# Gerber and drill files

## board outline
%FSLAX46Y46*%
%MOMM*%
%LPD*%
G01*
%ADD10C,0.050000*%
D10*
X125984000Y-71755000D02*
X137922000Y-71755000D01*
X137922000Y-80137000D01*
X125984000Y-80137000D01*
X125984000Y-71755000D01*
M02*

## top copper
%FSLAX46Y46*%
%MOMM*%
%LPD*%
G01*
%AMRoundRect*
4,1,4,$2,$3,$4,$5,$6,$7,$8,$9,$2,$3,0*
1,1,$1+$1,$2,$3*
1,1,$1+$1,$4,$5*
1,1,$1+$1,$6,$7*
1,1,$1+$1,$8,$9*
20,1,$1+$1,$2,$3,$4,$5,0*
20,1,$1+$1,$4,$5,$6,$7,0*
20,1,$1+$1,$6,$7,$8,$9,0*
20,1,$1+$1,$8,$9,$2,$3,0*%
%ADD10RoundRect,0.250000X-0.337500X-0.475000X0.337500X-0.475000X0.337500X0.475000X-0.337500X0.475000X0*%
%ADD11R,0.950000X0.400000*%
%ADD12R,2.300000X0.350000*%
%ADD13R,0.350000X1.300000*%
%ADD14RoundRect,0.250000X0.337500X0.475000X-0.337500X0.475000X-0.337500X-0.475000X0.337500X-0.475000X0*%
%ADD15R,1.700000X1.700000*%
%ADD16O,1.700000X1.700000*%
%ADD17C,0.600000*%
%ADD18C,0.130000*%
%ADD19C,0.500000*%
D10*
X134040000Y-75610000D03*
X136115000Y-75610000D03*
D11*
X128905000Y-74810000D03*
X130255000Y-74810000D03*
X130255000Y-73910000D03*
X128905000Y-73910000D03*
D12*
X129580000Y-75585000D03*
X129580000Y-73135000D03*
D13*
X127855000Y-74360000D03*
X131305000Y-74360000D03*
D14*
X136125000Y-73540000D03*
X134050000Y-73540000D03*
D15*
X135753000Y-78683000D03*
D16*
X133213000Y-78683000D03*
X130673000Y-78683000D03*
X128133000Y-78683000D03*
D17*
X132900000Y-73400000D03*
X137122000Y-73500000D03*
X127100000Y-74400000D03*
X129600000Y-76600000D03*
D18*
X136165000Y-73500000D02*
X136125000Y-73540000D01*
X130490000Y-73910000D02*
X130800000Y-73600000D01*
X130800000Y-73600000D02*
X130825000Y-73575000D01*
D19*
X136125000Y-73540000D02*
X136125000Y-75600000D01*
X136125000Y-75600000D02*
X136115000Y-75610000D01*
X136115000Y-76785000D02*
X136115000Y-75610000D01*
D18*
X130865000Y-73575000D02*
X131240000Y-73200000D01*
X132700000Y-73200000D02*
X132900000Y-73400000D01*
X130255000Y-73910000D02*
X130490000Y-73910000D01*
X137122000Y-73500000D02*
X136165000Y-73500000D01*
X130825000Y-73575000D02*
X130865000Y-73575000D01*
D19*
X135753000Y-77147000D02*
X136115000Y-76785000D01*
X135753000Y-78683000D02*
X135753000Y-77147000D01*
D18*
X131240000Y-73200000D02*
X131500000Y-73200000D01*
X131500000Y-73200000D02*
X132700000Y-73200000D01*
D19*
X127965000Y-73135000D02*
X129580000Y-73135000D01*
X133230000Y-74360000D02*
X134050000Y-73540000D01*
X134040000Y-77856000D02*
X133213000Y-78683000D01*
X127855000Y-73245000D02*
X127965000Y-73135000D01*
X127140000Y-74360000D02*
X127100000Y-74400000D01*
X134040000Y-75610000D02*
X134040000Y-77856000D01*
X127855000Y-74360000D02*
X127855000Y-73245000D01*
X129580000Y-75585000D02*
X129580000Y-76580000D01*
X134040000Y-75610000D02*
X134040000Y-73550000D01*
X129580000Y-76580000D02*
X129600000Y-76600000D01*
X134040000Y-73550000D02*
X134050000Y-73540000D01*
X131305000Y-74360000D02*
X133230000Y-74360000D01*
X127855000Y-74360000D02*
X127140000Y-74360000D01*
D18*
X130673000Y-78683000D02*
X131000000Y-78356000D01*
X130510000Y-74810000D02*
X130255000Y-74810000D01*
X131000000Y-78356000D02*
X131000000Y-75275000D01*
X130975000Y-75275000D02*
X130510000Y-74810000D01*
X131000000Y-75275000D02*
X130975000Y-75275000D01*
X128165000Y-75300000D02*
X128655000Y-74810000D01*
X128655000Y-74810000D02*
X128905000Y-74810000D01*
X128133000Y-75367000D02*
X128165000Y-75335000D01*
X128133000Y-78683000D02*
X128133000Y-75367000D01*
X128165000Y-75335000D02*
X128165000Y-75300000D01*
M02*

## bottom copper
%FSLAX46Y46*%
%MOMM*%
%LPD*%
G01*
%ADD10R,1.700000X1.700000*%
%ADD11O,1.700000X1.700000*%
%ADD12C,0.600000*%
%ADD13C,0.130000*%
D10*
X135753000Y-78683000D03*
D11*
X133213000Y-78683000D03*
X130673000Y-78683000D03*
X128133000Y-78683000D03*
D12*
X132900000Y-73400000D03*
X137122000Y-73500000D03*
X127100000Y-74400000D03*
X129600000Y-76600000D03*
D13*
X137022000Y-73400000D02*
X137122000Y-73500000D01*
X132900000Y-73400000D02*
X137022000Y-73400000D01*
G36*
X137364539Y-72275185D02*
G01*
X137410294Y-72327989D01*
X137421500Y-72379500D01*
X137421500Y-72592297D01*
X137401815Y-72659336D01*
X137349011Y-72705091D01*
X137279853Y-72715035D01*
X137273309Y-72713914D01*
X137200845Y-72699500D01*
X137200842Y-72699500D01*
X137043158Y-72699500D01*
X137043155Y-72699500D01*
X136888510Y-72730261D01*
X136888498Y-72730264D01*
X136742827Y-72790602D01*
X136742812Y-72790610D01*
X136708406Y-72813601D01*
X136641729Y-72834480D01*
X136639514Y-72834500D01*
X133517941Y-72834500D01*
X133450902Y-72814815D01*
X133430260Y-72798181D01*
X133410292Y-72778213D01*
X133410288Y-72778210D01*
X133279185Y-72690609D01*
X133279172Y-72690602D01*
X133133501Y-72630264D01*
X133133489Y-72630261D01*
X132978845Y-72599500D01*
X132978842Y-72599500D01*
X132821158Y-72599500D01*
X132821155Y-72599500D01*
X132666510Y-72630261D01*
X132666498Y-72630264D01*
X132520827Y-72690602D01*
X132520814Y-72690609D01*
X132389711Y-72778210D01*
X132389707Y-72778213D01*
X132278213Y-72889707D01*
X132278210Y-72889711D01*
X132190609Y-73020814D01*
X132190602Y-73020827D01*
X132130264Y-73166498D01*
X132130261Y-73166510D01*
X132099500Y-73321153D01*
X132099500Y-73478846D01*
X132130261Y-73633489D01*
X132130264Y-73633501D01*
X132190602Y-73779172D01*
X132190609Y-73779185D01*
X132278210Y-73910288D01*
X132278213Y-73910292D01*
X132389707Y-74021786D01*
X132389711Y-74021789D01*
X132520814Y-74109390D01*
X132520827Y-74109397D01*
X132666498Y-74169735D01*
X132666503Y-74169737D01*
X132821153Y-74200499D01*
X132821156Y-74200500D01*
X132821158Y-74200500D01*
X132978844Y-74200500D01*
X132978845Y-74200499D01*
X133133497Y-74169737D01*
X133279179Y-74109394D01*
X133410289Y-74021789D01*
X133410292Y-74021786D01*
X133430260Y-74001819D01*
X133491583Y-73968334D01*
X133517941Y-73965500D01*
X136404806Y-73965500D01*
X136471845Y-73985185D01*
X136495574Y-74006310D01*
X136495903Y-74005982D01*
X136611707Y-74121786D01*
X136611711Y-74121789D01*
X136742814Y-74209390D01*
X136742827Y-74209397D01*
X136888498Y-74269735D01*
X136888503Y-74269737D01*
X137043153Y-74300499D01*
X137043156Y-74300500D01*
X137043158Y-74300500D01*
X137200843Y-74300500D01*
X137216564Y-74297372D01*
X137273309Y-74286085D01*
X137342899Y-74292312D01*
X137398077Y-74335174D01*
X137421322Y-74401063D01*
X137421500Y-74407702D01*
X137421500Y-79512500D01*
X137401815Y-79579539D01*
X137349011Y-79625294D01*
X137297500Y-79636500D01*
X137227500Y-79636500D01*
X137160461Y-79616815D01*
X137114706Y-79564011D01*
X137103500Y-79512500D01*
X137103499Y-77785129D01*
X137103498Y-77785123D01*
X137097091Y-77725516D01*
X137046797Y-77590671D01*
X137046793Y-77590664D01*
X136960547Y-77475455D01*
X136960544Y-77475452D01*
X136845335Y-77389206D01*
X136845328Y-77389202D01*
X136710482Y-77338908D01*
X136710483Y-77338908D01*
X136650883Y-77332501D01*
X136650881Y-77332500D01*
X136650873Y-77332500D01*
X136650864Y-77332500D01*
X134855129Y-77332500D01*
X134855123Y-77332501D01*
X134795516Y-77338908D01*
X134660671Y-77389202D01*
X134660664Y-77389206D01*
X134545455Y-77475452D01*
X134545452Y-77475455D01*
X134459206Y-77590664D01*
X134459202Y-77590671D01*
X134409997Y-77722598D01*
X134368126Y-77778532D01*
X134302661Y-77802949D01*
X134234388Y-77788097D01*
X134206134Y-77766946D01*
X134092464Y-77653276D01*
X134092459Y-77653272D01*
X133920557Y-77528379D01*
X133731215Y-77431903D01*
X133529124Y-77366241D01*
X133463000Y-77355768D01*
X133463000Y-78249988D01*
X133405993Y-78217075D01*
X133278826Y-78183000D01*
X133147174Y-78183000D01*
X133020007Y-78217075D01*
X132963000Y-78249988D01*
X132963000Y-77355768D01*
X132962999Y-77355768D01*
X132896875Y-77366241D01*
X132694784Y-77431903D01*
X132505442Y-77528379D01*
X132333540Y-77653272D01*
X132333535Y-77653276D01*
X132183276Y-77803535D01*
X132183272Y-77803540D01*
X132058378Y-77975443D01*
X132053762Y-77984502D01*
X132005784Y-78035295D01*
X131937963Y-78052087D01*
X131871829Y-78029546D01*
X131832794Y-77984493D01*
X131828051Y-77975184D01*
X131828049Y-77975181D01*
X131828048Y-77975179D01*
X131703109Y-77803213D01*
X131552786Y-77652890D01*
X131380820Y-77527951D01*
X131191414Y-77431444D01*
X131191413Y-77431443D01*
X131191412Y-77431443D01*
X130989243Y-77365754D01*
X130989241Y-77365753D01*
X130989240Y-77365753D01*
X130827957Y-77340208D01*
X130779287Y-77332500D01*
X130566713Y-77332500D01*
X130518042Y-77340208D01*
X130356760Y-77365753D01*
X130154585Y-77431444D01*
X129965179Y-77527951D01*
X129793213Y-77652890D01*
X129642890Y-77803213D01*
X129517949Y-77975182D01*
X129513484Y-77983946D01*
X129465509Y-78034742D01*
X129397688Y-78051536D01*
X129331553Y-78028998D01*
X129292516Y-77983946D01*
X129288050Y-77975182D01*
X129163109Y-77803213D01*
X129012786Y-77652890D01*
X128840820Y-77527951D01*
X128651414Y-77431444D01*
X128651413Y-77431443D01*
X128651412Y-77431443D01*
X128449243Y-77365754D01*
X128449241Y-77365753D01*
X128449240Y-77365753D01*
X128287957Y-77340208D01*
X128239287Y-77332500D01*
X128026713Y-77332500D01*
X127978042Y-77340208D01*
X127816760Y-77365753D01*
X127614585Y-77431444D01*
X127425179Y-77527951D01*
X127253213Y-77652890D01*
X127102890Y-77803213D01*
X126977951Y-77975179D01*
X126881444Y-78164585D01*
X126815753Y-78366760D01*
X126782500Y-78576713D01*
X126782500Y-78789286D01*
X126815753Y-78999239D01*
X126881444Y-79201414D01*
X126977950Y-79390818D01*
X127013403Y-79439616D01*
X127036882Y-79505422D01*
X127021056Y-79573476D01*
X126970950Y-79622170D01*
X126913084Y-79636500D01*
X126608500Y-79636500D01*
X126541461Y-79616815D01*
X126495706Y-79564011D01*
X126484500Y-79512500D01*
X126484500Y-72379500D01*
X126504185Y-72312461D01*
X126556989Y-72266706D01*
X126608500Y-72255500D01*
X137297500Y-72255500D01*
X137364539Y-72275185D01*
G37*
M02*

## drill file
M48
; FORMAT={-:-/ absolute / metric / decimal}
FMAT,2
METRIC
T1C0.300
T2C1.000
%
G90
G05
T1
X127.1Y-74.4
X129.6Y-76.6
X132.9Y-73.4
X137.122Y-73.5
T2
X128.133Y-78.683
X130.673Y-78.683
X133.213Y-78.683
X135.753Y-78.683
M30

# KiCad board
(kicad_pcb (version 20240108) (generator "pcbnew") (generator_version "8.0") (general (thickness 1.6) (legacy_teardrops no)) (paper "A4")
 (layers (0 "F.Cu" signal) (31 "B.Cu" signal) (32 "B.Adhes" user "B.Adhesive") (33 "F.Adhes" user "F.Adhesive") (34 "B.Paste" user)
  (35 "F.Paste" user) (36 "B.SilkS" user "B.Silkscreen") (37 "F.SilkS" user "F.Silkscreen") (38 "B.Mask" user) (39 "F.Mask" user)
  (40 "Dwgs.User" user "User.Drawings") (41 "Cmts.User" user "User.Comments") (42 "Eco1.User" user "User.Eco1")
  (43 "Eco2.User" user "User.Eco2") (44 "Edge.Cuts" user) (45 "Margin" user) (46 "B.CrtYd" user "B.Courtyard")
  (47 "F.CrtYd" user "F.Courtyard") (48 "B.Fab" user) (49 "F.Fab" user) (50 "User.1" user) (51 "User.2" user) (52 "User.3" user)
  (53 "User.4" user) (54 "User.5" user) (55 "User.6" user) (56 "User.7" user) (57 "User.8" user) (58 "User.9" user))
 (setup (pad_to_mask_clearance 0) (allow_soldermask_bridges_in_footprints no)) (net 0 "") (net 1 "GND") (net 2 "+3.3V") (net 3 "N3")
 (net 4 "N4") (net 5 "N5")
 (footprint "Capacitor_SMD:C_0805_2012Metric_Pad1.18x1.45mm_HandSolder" (layer "F.Cu") (at 135.0775 75.61)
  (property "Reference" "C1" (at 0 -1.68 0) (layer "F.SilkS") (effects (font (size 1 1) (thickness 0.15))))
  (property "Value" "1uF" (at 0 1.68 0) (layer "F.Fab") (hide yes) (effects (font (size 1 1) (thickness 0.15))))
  (pad "1" smd roundrect (at -1.0375 0) (size 1.175 1.45) (layers "F.Cu" "F.Paste" "F.Mask") (roundrect_rratio 0.212766) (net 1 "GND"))
  (pad "2" smd roundrect (at 1.0375 0) (size 1.175 1.45) (layers "F.Cu" "F.Paste" "F.Mask") (roundrect_rratio 0.212766) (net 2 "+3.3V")))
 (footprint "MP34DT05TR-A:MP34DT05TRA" (layer "F.Cu") (at 129.58 74.36 90)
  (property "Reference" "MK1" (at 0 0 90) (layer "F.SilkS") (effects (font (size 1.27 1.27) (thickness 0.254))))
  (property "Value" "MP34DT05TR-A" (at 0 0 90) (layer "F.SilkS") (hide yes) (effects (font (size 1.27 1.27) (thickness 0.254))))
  (pad "1" smd rect (at -0.45 -0.675 90) (size 0.4 0.95) (layers "F.Cu" "F.Paste" "F.Mask") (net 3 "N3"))
  (pad "2" smd rect (at -0.45 0.675 90) (size 0.4 0.95) (layers "F.Cu" "F.Paste" "F.Mask") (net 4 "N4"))
  (pad "3" smd rect (at 0.45 0.675 90) (size 0.4 0.95) (layers "F.Cu" "F.Paste" "F.Mask") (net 2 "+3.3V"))
  (pad "4" smd rect (at 0.45 -0.675 90) (size 0.4 0.95) (layers "F.Cu" "F.Paste" "F.Mask") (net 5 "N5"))
  (pad "5" smd rect (at -1.225 0 90) (size 0.35 2.3) (layers "F.Cu" "F.Paste" "F.Mask") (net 1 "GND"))
  (pad "6" smd rect (at 1.225 0 90) (size 0.35 2.3) (layers "F.Cu" "F.Paste" "F.Mask") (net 1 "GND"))
  (pad "7" smd rect (at 0 -1.725 180) (size 0.35 1.3) (layers "F.Cu" "F.Paste" "F.Mask") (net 1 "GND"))
  (pad "8" smd rect (at 0 1.725 180) (size 0.35 1.3) (layers "F.Cu" "F.Paste" "F.Mask") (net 1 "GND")))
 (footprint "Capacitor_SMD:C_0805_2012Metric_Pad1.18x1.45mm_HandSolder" (layer "F.Cu") (at 135.0875 73.54 180)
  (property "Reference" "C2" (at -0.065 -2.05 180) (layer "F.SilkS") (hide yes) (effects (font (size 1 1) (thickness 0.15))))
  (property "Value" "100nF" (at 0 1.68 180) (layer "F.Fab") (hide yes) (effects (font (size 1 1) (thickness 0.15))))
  (pad "1" smd roundrect (at -1.0375 0 180) (size 1.175 1.45) (layers "F.Cu" "F.Paste" "F.Mask") (roundrect_rratio 0.212766) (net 2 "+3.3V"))
  (pad "2" smd roundrect (at 1.0375 0 180) (size 1.175 1.45) (layers "F.Cu" "F.Paste" "F.Mask") (roundrect_rratio 0.212766) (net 1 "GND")))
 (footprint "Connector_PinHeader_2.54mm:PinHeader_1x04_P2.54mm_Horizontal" (layer "F.Cu") (at 135.753 78.683 -90)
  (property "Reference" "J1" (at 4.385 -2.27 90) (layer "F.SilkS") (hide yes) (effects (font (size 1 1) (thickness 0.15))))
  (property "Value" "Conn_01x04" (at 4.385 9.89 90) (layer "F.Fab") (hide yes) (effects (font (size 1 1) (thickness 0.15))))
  (pad "1" thru_hole rect (at 0 0 270) (size 1.7 1.7) (drill 1) (layers "*.Cu" "*.Mask") (remove_unused_layers no) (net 2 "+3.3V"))
  (pad "2" thru_hole oval (at 0 2.54 270) (size 1.7 1.7) (drill 1) (layers "*.Cu" "*.Mask") (remove_unused_layers no) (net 1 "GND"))
  (pad "3" thru_hole oval (at 0 5.08 270) (size 1.7 1.7) (drill 1) (layers "*.Cu" "*.Mask") (remove_unused_layers no) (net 4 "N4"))
  (pad "4" thru_hole oval (at 0 7.62 270) (size 1.7 1.7) (drill 1) (layers "*.Cu" "*.Mask") (remove_unused_layers no) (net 3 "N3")))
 (gr_rect (start 125.984 71.755) (end 137.922 80.137) (stroke (width 0.05) (type default)) (fill none) (layer "Edge.Cuts"))
 (segment (start 136.165 73.5) (end 136.125 73.54) (width 0.13) (layer "F.Cu") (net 2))
 (segment (start 130.49 73.91) (end 130.8 73.6) (width 0.13) (layer "F.Cu") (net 2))
 (segment (start 130.8 73.6) (end 130.825 73.575) (width 0.13) (layer "F.Cu") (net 2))
 (segment (start 136.125 73.54) (end 136.125 75.6) (width 0.5) (layer "F.Cu") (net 2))
 (segment (start 136.125 75.6) (end 136.115 75.61) (width 0.5) (layer "F.Cu") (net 2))
 (segment (start 136.115 76.785) (end 136.115 75.61) (width 0.5) (layer "F.Cu") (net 2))
 (segment (start 130.865 73.575) (end 131.24 73.2) (width 0.13) (layer "F.Cu") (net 2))
 (segment (start 132.7 73.2) (end 132.9 73.4) (width 0.13) (layer "F.Cu") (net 2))
 (segment (start 130.255 73.91) (end 130.49 73.91) (width 0.13) (layer "F.Cu") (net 2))
 (segment (start 137.122 73.5) (end 136.165 73.5) (width 0.13) (layer "F.Cu") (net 2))
 (segment (start 130.825 73.575) (end 130.865 73.575) (width 0.13) (layer "F.Cu") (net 2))
 (segment (start 135.753 77.147) (end 136.115 76.785) (width 0.5) (layer "F.Cu") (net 2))
 (segment (start 135.753 78.683) (end 135.753 77.147) (width 0.5) (layer "F.Cu") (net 2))
 (segment (start 131.24 73.2) (end 131.5 73.2) (width 0.13) (layer "F.Cu") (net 2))
 (segment (start 131.5 73.2) (end 132.7 73.2) (width 0.13) (layer "F.Cu") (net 2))
 (via (at 132.9 73.4) (size 0.6) (drill 0.3) (layers "F.Cu" "B.Cu") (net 2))
 (via (at 137.122 73.5) (size 0.6) (drill 0.3) (layers "F.Cu" "B.Cu") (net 2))
 (segment (start 137.022 73.4) (end 137.122 73.5) (width 0.13) (layer "B.Cu") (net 2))
 (segment (start 132.9 73.4) (end 137.022 73.4) (width 0.13) (layer "B.Cu") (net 2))
 (segment (start 127.965 73.135) (end 129.58 73.135) (width 0.5) (layer "F.Cu") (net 1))
 (segment (start 133.23 74.36) (end 134.05 73.54) (width 0.5) (layer "F.Cu") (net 1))
 (segment (start 134.04 77.856) (end 133.213 78.683) (width 0.5) (layer "F.Cu") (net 1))
 (segment (start 127.855 73.245) (end 127.965 73.135) (width 0.5) (layer "F.Cu") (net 1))
 (segment (start 127.14 74.36) (end 127.1 74.4) (width 0.5) (layer "F.Cu") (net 1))
 (segment (start 134.04 75.61) (end 134.04 77.856) (width 0.5) (layer "F.Cu") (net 1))
 (segment (start 127.855 74.36) (end 127.855 73.245) (width 0.5) (layer "F.Cu") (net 1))
 (segment (start 129.58 75.585) (end 129.58 76.58) (width 0.5) (layer "F.Cu") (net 1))
 (segment (start 134.04 75.61) (end 134.04 73.55) (width 0.5) (layer "F.Cu") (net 1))
 (segment (start 129.58 76.58) (end 129.6 76.6) (width 0.5) (layer "F.Cu") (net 1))
 (segment (start 134.04 73.55) (end 134.05 73.54) (width 0.5) (layer "F.Cu") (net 1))
 (segment (start 131.305 74.36) (end 133.23 74.36) (width 0.5) (layer "F.Cu") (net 1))
 (segment (start 127.855 74.36) (end 127.14 74.36) (width 0.5) (layer "F.Cu") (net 1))
 (via (at 127.1 74.4) (size 0.6) (drill 0.3) (layers "F.Cu" "B.Cu") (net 1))
 (via (at 129.6 76.6) (size 0.6) (drill 0.3) (layers "F.Cu" "B.Cu") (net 1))
 (segment (start 130.673 78.683) (end 131 78.356) (width 0.13) (layer "F.Cu") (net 4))
 (segment (start 130.51 74.81) (end 130.255 74.81) (width 0.13) (layer "F.Cu") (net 4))
 (segment (start 131 78.356) (end 131 75.275) (width 0.13) (layer "F.Cu") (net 4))
 (segment (start 130.975 75.275) (end 130.51 74.81) (width 0.13) (layer "F.Cu") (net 4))
 (segment (start 131 75.275) (end 130.975 75.275) (width 0.13) (layer "F.Cu") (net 4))
 (segment (start 128.165 75.3) (end 128.655 74.81) (width 0.13) (layer "F.Cu") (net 3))
 (segment (start 128.655 74.81) (end 128.905 74.81) (width 0.13) (layer "F.Cu") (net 3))
 (segment (start 128.133 75.367) (end 128.165 75.335) (width 0.13) (layer "F.Cu") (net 3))
 (segment (start 128.133 78.683) (end 128.133 75.367) (width 0.13) (layer "F.Cu") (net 3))
 (segment (start 128.165 75.335) (end 128.165 75.3) (width 0.13) (layer "F.Cu") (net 3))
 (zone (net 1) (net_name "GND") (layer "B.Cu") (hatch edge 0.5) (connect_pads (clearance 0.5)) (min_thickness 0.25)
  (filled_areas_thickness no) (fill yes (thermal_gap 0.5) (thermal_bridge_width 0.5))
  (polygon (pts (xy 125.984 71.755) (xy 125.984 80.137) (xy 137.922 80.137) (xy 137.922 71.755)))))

